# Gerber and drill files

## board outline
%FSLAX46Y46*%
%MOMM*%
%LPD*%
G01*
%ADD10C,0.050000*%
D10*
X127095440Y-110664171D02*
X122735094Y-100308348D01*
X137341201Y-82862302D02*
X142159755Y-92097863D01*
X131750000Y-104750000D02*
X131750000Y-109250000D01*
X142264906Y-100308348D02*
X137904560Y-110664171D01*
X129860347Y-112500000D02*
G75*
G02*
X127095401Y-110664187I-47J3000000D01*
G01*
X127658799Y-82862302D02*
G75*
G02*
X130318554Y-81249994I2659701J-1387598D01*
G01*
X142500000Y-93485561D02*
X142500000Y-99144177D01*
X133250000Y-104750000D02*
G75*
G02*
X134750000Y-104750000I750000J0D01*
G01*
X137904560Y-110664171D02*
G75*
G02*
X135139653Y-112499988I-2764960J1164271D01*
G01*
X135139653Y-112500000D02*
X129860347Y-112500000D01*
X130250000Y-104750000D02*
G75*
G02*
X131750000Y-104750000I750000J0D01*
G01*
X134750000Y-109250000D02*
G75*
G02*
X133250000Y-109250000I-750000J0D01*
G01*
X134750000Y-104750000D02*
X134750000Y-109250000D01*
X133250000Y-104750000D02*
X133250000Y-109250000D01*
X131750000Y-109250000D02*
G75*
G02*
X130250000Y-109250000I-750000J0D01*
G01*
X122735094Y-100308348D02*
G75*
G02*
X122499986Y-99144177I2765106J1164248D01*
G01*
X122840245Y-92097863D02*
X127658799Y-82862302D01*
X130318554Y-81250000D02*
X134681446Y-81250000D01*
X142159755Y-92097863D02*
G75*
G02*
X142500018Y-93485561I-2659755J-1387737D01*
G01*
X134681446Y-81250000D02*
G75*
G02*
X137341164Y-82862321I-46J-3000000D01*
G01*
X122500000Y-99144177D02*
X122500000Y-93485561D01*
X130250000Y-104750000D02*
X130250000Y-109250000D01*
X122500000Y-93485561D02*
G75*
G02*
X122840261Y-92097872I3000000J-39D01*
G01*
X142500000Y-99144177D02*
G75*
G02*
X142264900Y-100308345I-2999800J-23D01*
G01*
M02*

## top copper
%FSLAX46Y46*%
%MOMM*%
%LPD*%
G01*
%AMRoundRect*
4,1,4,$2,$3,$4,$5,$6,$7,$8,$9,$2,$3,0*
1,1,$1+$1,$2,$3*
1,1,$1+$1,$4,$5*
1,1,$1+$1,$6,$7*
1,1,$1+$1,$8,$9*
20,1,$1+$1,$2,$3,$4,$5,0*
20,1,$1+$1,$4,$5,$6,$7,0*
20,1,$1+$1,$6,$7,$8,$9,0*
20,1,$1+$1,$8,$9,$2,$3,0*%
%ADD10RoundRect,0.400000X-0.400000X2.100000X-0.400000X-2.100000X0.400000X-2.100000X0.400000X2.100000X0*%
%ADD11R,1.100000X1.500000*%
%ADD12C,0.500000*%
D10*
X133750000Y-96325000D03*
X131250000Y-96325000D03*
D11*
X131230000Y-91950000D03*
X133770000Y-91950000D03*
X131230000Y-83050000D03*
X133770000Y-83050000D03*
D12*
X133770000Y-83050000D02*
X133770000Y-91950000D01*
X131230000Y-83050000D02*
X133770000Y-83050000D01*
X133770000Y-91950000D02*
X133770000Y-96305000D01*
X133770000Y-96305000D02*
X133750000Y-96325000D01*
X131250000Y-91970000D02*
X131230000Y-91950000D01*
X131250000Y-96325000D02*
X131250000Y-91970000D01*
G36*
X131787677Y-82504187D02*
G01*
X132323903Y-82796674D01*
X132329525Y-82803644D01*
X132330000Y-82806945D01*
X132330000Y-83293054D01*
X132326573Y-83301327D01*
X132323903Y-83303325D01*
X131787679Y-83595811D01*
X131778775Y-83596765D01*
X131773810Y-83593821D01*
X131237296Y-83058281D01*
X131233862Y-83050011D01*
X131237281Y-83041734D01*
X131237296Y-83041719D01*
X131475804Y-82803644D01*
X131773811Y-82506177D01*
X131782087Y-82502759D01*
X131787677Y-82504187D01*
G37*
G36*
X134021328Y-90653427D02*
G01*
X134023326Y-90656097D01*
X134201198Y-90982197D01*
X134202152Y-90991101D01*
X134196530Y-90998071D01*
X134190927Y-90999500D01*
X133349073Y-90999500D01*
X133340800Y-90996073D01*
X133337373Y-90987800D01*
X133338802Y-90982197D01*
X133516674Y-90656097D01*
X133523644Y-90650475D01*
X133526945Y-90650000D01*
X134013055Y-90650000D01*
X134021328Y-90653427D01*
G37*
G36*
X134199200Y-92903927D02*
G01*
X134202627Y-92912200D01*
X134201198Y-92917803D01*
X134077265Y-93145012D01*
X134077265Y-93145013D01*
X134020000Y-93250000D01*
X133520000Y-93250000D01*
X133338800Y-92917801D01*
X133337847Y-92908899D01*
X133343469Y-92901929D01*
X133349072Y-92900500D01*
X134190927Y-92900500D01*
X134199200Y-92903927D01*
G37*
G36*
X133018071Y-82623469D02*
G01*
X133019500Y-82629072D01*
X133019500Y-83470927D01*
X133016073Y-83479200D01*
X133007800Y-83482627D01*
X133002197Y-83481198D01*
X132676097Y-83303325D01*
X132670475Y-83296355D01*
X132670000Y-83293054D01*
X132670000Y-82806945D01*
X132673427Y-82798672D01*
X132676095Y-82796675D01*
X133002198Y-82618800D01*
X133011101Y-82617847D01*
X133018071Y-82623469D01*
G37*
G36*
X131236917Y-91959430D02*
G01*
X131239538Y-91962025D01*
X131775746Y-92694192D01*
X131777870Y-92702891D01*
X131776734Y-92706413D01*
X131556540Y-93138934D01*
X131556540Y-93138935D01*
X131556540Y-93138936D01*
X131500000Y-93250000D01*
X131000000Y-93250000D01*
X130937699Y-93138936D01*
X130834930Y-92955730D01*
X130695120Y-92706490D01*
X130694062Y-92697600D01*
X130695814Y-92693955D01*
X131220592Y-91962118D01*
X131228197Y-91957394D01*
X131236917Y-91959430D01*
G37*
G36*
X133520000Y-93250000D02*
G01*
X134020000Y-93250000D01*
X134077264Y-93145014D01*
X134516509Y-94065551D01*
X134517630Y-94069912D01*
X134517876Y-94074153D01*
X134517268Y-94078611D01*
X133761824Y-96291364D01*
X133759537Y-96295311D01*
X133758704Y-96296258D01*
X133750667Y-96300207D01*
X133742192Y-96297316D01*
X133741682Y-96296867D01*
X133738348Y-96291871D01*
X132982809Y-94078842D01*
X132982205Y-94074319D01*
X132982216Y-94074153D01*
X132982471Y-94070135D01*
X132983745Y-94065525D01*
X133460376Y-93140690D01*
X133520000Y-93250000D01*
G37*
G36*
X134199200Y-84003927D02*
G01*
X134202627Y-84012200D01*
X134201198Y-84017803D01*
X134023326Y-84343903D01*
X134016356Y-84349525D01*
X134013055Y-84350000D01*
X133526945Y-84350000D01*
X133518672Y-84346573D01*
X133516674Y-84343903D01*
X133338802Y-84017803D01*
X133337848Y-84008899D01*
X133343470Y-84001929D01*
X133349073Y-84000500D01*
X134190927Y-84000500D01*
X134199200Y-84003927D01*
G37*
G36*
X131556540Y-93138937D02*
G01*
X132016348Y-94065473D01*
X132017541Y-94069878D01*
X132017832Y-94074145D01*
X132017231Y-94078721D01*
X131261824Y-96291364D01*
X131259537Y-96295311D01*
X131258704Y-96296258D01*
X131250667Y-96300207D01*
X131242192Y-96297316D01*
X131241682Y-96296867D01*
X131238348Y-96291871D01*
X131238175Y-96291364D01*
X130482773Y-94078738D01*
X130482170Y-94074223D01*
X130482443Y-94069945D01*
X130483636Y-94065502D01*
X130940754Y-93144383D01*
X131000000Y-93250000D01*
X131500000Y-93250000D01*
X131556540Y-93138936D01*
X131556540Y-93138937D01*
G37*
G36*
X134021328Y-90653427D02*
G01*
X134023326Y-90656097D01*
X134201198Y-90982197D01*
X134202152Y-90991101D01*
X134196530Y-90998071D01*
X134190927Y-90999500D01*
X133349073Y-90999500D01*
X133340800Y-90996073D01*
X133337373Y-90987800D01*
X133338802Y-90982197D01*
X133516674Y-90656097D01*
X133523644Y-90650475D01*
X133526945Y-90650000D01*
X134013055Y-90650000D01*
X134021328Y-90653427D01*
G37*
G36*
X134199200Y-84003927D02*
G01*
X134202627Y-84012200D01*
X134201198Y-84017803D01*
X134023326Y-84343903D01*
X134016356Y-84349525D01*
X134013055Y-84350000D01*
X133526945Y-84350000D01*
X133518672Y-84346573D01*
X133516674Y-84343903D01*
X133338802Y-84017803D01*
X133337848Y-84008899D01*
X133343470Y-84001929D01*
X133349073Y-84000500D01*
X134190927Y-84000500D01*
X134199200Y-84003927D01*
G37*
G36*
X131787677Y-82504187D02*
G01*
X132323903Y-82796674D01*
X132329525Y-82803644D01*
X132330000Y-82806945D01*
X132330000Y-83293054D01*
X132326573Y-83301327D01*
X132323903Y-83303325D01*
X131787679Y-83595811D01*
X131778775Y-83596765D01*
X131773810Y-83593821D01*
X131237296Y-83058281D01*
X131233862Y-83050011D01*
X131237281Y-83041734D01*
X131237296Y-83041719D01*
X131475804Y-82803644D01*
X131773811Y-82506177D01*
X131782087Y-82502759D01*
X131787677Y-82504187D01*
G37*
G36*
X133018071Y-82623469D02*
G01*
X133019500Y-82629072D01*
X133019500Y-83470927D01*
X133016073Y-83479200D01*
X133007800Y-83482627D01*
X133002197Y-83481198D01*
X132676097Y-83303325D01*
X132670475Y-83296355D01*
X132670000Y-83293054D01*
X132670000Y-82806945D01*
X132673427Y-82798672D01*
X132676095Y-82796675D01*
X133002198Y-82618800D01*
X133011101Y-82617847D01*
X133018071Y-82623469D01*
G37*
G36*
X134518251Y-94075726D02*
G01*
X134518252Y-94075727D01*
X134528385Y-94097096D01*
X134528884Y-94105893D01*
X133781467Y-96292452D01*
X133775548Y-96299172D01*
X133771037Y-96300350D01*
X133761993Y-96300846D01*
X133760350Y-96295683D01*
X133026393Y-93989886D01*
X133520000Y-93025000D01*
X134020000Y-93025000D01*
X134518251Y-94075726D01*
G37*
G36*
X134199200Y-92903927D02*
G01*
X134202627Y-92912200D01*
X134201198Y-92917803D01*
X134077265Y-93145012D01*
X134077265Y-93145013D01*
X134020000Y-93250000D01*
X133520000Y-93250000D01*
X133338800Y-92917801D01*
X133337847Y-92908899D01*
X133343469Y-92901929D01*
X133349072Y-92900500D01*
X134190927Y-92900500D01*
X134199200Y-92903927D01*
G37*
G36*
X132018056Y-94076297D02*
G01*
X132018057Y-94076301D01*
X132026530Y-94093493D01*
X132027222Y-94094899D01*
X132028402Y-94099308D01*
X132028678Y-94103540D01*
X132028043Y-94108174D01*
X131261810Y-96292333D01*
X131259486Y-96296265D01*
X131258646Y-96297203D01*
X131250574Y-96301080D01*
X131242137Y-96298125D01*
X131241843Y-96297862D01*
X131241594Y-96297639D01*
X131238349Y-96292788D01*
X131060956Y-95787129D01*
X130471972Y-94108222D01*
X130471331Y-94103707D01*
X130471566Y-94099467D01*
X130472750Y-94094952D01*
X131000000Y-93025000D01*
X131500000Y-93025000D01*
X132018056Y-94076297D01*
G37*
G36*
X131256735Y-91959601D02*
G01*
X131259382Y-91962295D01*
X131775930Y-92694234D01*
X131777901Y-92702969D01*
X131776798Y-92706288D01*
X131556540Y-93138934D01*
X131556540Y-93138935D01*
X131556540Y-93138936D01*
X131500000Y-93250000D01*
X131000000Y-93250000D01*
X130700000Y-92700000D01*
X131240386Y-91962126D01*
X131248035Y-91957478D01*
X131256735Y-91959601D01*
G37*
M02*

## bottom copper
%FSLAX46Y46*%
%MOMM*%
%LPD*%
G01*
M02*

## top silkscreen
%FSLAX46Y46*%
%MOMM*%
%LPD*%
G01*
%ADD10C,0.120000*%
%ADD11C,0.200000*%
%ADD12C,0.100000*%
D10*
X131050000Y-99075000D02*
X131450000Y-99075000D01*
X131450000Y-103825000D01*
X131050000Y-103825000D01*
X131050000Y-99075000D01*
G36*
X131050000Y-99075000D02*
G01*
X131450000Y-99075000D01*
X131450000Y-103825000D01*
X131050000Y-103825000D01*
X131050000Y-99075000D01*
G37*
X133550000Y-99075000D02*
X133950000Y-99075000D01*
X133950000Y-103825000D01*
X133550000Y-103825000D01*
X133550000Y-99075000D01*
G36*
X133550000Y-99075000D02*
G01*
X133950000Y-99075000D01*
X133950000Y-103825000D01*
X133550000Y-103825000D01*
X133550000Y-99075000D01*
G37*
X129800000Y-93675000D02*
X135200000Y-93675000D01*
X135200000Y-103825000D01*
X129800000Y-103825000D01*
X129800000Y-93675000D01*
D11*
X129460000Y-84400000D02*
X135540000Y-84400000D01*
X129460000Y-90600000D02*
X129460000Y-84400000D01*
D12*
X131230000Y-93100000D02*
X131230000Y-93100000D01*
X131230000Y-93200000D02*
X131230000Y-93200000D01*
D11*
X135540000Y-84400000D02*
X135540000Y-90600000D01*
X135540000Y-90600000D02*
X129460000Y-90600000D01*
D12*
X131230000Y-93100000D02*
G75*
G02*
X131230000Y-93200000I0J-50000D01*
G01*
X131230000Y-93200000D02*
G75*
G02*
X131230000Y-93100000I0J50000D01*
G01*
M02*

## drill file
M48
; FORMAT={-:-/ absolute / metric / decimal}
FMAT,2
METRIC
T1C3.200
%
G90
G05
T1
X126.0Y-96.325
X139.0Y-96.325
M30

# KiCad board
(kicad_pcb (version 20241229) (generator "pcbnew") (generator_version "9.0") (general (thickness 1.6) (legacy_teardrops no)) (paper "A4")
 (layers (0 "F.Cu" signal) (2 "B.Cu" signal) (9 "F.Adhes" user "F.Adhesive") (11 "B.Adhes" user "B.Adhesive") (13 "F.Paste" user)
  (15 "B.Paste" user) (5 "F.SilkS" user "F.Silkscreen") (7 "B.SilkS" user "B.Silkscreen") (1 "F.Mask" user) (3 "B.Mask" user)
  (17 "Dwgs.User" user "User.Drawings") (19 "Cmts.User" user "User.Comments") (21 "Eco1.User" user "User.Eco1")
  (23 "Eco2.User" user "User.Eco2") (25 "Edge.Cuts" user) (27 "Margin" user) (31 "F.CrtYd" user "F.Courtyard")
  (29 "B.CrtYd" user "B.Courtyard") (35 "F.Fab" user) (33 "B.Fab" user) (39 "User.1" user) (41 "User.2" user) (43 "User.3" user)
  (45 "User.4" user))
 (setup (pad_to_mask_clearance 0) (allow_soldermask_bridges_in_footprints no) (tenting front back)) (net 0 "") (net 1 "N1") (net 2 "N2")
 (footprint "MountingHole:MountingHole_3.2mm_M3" (layer "F.Cu") (at 139 96.325)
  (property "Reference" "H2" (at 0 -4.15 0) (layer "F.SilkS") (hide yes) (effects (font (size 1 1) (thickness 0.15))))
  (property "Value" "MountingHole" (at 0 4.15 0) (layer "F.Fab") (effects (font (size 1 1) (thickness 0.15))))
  (pad "" np_thru_hole circle (at 0 0) (size 3.2 3.2) (drill 3.2) (layers "*.Cu" "*.Mask")))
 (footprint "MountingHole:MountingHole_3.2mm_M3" (layer "F.Cu") (at 126 96.325)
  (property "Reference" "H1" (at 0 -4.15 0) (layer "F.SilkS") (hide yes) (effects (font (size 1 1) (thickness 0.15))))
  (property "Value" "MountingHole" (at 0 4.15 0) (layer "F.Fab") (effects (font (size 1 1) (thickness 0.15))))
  (pad "" np_thru_hole circle (at 0 0) (size 3.2 3.2) (drill 3.2) (layers "*.Cu" "*.Mask")))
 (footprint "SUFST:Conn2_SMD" (layer "F.Cu") (at 132.5 96.325 180)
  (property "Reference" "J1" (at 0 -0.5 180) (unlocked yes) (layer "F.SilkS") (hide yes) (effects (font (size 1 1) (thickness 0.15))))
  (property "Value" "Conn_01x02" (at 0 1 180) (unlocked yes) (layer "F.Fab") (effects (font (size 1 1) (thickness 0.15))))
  (fp_rect (start 1.05 -7.5) (end 1.45 -2.75) (stroke (width 0.12) (type solid)) (fill yes) (layer "F.SilkS"))
  (fp_rect (start -1.45 -7.5) (end -1.05 -2.75) (stroke (width 0.12) (type solid)) (fill yes) (layer "F.SilkS"))
  (fp_rect (start -2.7 -7.5) (end 2.7 2.65) (stroke (width 0.12) (type default)) (fill no) (layer "F.SilkS"))
  (pad "1" smd roundrect (at -1.25 0 270) (size 5 1.6) (layers "F.Cu" "F.Mask" "F.Paste") (roundrect_rratio 0.25) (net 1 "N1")
   (thermal_bridge_angle 45)
   (teardrops (best_length_ratio 0.5) (max_length 1) (best_width_ratio 1) (max_width 2) (curved_edges no) (filter_ratio 0.9) (enabled yes)
    (allow_two_segments yes) (prefer_zone_connections yes)))
  (pad "2" smd roundrect (at 1.25 0 270) (size 5 1.6) (layers "F.Cu" "F.Mask" "F.Paste") (roundrect_rratio 0.25) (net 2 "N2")
   (thermal_bridge_angle 45)
   (teardrops (best_length_ratio 0.5) (max_length 1) (best_width_ratio 1) (max_width 2) (curved_edges no) (filter_ratio 0.9) (enabled yes)
    (allow_two_segments yes) (prefer_zone_connections yes))))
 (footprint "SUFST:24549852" (layer "F.Cu") (at 132.5 87.5)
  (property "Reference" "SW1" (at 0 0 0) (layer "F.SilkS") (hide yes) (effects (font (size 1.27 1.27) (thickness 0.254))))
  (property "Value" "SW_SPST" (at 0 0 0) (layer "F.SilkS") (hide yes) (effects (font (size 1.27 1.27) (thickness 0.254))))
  (fp_line (start -3.04 -3.1) (end 3.04 -3.1) (stroke (width 0.2) (type solid)) (layer "F.SilkS"))
  (fp_line (start -3.04 3.1) (end -3.04 -3.1) (stroke (width 0.2) (type solid)) (layer "F.SilkS"))
  (fp_line (start -1.27 5.6) (end -1.27 5.6) (stroke (width 0.1) (type solid)) (layer "F.SilkS"))
  (fp_line (start -1.27 5.7) (end -1.27 5.7) (stroke (width 0.1) (type solid)) (layer "F.SilkS"))
  (fp_line (start 3.04 -3.1) (end 3.04 3.1) (stroke (width 0.2) (type solid)) (layer "F.SilkS"))
  (fp_line (start 3.04 3.1) (end -3.04 3.1) (stroke (width 0.2) (type solid)) (layer "F.SilkS"))
  (fp_arc (start -1.27 5.6) (mid -1.22 5.65) (end -1.27 5.7) (stroke (width 0.1) (type solid)) (layer "F.SilkS"))
  (fp_arc (start -1.27 5.7) (mid -1.32 5.65) (end -1.27 5.6) (stroke (width 0.1) (type solid)) (layer "F.SilkS"))
  (pad "A1" smd rect (at -1.27 4.45) (size 1.1 1.5) (layers "F.Cu" "F.Mask" "F.Paste") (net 2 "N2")
   (teardrops (best_length_ratio 0.5) (max_length 1) (best_width_ratio 1) (max_width 2) (curved_edges no) (filter_ratio 0.9) (enabled yes)
    (allow_two_segments yes) (prefer_zone_connections yes)))
  (pad "A2" smd rect (at 1.27 4.45) (size 1.1 1.5) (layers "F.Cu" "F.Mask" "F.Paste")
   (teardrops (best_length_ratio 0.5) (max_length 1) (best_width_ratio 1) (max_width 2) (curved_edges no) (filter_ratio 0.9) (enabled yes)
    (allow_two_segments yes) (prefer_zone_connections yes)))
  (pad "B1" smd rect (at -1.27 -4.45) (size 1.1 1.5) (layers "F.Cu" "F.Mask" "F.Paste") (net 1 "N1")
   (teardrops (best_length_ratio 0.5) (max_length 1) (best_width_ratio 1) (max_width 2) (curved_edges no) (filter_ratio 0.9) (enabled yes)
    (allow_two_segments yes) (prefer_zone_connections yes)))
  (pad "B2" smd rect (at 1.27 -4.45) (size 1.1 1.5) (layers "F.Cu" "F.Mask" "F.Paste")
   (teardrops (best_length_ratio 0.5) (max_length 1) (best_width_ratio 1) (max_width 2) (curved_edges no) (filter_ratio 0.9) (enabled yes)
    (allow_two_segments yes) (prefer_zone_connections yes))))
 (gr_line (start 127.09544 110.664171) (end 122.735094 100.308348) (stroke (width 0.05) (type default)) (layer "Edge.Cuts"))
 (gr_line (start 137.341201 82.862302) (end 142.159755 92.097863) (stroke (width 0.05) (type default)) (layer "Edge.Cuts"))
 (gr_line (start 131.75 104.75) (end 131.75 109.25) (stroke (width 0.05) (type default)) (layer "Edge.Cuts"))
 (gr_line (start 142.264906 100.308348) (end 137.90456 110.664171) (stroke (width 0.05) (type default)) (layer "Edge.Cuts"))
 (gr_arc (start 129.860347 112.5) (mid 128.200906 111.999251) (end 127.09544 110.664171) (stroke (width 0.05) (type default))
  (layer "Edge.Cuts"))
 (gr_arc (start 127.658799 82.862302) (mid 128.763412 81.68453) (end 130.318554 81.25) (stroke (width 0.05) (type default))
  (layer "Edge.Cuts"))
 (gr_line (start 142.5 93.485561) (end 142.5 99.144177) (stroke (width 0.05) (type default)) (layer "Edge.Cuts"))
 (gr_arc (start 133.25 104.75) (mid 134 104) (end 134.75 104.75) (stroke (width 0.05) (type default)) (layer "Edge.Cuts"))
 (gr_arc (start 137.90456 110.664171) (mid 136.79909 111.999234) (end 135.139653 112.5) (stroke (width 0.05) (type default))
  (layer "Edge.Cuts"))
 (gr_line (start 135.139653 112.5) (end 129.860347 112.5) (stroke (width 0.05) (type default)) (layer "Edge.Cuts"))
 (gr_arc (start 130.25 104.75) (mid 131 104) (end 131.75 104.75) (stroke (width 0.05) (type default)) (layer "Edge.Cuts"))
 (gr_arc (start 134.75 109.25) (mid 134 110) (end 133.25 109.25) (stroke (width 0.05) (type default)) (layer "Edge.Cuts"))
 (gr_line (start 134.75 104.75) (end 134.75 109.25) (stroke (width 0.05) (type default)) (layer "Edge.Cuts"))
 (gr_line (start 133.25 104.75) (end 133.25 109.25) (stroke (width 0.05) (type default)) (layer "Edge.Cuts"))
 (gr_arc (start 131.75 109.25) (mid 131 110) (end 130.25 109.25) (stroke (width 0.05) (type default)) (layer "Edge.Cuts"))
 (gr_arc (start 122.735094 100.308348) (mid 122.559365 99.738012) (end 122.5 99.144177) (stroke (width 0.05) (type default))
  (layer "Edge.Cuts"))
 (gr_line (start 122.840245 92.097863) (end 127.658799 82.862302) (stroke (width 0.05) (type default)) (layer "Edge.Cuts"))
 (gr_line (start 130.318554 81.25) (end 134.681446 81.25) (stroke (width 0.05) (type default)) (layer "Edge.Cuts"))
 (gr_arc (start 142.159755 92.097863) (mid 142.413698 92.77116) (end 142.5 93.485561) (stroke (width 0.05) (type default))
  (layer "Edge.Cuts"))
 (gr_arc (start 134.681446 81.25) (mid 136.236584 81.684547) (end 137.341201 82.862302) (stroke (width 0.05) (type default))
  (layer "Edge.Cuts"))
 (gr_line (start 122.5 99.144177) (end 122.5 93.485561) (stroke (width 0.05) (type default)) (layer "Edge.Cuts"))
 (gr_line (start 130.25 104.75) (end 130.25 109.25) (stroke (width 0.05) (type default)) (layer "Edge.Cuts"))
 (gr_arc (start 122.5 93.485561) (mid 122.586303 92.771161) (end 122.840245 92.097863) (stroke (width 0.05) (type default))
  (layer "Edge.Cuts"))
 (gr_arc (start 142.5 99.144177) (mid 142.440644 99.738014) (end 142.264906 100.308348) (stroke (width 0.05) (type default))
  (layer "Edge.Cuts"))
 (segment (start 133.77 83.05) (end 133.77 91.95) (width 0.5) (layer "F.Cu") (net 1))
 (segment (start 131.23 83.05) (end 133.77 83.05) (width 0.5) (layer "F.Cu") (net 1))
 (segment (start 133.77 91.95) (end 133.77 96.305) (width 0.5) (layer "F.Cu") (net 1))
 (segment (start 133.77 96.305) (end 133.75 96.325) (width 0.5) (layer "F.Cu") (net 1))
 (segment (start 131.25 91.97) (end 131.23 91.95) (width 0.5) (layer "F.Cu") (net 2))
 (segment (start 131.25 96.325) (end 131.25 91.97) (width 0.5) (layer "F.Cu") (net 2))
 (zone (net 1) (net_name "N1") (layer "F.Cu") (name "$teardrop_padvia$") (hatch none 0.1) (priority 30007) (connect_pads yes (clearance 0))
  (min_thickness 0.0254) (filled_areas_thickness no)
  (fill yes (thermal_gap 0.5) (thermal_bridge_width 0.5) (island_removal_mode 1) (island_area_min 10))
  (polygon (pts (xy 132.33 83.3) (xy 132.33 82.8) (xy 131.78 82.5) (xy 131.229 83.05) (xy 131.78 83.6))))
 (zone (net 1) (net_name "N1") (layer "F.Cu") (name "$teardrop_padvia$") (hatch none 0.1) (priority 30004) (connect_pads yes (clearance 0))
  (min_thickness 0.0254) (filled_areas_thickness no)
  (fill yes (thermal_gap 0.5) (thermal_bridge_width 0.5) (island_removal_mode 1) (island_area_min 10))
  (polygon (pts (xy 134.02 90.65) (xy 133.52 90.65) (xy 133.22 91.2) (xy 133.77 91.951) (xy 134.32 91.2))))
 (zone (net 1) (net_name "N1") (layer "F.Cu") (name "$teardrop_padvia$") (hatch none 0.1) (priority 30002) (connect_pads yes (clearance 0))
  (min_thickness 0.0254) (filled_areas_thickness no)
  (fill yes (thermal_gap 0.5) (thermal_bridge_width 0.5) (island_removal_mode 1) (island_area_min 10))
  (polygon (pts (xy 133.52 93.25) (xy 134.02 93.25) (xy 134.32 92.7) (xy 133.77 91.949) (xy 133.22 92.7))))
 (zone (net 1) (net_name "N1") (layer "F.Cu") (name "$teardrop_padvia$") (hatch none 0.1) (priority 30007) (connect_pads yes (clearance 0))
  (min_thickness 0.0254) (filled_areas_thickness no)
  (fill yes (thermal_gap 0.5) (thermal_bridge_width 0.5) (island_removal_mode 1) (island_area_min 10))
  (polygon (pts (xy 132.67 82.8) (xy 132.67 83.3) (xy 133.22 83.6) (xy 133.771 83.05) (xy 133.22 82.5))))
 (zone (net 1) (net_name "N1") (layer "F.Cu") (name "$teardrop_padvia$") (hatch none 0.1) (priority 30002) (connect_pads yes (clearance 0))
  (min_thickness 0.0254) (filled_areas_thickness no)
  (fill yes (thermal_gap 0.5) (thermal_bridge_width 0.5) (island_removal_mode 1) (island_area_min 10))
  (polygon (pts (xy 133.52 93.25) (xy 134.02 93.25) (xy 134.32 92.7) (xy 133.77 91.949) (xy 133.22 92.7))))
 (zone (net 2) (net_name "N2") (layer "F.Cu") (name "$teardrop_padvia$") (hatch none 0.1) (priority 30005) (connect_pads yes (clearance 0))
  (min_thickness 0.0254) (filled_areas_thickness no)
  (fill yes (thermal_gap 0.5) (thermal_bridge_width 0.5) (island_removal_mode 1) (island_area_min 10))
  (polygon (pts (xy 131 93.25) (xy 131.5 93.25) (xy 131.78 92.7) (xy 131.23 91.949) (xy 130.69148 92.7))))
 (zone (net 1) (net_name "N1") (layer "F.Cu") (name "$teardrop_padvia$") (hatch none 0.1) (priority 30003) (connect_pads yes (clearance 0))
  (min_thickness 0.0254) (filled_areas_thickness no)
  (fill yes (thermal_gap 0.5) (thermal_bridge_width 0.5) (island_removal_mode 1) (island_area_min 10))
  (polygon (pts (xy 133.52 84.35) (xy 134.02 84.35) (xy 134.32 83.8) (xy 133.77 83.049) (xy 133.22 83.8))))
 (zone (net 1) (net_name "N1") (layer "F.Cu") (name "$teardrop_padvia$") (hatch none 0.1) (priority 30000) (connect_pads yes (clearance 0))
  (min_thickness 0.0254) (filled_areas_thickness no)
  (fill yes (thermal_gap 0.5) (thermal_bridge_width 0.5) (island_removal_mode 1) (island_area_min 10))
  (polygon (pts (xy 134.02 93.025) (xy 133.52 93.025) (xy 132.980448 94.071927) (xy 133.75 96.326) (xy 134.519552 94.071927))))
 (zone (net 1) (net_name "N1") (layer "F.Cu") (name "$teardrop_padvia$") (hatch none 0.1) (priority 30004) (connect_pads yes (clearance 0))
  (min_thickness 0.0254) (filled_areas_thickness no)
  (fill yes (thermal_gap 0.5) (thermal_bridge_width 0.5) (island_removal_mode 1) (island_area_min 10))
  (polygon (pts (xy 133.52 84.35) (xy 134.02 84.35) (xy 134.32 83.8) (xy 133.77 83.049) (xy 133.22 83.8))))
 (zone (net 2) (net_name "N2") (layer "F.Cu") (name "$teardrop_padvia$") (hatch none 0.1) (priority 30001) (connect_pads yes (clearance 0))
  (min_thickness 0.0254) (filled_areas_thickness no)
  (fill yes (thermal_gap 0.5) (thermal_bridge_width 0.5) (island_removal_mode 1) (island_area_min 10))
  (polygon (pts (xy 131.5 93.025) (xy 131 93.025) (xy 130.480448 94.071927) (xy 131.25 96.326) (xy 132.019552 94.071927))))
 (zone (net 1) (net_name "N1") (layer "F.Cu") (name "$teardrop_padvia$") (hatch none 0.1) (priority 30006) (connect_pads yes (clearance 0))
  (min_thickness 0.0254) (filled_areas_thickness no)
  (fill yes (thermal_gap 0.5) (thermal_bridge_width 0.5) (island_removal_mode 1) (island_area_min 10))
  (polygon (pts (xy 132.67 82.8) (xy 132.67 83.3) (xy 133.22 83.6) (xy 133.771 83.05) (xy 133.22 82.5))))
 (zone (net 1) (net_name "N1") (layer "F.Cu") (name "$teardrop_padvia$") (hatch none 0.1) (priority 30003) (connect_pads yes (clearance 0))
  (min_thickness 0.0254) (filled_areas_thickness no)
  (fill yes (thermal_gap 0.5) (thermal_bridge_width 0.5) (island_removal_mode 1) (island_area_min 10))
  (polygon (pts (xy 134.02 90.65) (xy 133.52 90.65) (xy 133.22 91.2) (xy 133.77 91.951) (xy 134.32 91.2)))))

